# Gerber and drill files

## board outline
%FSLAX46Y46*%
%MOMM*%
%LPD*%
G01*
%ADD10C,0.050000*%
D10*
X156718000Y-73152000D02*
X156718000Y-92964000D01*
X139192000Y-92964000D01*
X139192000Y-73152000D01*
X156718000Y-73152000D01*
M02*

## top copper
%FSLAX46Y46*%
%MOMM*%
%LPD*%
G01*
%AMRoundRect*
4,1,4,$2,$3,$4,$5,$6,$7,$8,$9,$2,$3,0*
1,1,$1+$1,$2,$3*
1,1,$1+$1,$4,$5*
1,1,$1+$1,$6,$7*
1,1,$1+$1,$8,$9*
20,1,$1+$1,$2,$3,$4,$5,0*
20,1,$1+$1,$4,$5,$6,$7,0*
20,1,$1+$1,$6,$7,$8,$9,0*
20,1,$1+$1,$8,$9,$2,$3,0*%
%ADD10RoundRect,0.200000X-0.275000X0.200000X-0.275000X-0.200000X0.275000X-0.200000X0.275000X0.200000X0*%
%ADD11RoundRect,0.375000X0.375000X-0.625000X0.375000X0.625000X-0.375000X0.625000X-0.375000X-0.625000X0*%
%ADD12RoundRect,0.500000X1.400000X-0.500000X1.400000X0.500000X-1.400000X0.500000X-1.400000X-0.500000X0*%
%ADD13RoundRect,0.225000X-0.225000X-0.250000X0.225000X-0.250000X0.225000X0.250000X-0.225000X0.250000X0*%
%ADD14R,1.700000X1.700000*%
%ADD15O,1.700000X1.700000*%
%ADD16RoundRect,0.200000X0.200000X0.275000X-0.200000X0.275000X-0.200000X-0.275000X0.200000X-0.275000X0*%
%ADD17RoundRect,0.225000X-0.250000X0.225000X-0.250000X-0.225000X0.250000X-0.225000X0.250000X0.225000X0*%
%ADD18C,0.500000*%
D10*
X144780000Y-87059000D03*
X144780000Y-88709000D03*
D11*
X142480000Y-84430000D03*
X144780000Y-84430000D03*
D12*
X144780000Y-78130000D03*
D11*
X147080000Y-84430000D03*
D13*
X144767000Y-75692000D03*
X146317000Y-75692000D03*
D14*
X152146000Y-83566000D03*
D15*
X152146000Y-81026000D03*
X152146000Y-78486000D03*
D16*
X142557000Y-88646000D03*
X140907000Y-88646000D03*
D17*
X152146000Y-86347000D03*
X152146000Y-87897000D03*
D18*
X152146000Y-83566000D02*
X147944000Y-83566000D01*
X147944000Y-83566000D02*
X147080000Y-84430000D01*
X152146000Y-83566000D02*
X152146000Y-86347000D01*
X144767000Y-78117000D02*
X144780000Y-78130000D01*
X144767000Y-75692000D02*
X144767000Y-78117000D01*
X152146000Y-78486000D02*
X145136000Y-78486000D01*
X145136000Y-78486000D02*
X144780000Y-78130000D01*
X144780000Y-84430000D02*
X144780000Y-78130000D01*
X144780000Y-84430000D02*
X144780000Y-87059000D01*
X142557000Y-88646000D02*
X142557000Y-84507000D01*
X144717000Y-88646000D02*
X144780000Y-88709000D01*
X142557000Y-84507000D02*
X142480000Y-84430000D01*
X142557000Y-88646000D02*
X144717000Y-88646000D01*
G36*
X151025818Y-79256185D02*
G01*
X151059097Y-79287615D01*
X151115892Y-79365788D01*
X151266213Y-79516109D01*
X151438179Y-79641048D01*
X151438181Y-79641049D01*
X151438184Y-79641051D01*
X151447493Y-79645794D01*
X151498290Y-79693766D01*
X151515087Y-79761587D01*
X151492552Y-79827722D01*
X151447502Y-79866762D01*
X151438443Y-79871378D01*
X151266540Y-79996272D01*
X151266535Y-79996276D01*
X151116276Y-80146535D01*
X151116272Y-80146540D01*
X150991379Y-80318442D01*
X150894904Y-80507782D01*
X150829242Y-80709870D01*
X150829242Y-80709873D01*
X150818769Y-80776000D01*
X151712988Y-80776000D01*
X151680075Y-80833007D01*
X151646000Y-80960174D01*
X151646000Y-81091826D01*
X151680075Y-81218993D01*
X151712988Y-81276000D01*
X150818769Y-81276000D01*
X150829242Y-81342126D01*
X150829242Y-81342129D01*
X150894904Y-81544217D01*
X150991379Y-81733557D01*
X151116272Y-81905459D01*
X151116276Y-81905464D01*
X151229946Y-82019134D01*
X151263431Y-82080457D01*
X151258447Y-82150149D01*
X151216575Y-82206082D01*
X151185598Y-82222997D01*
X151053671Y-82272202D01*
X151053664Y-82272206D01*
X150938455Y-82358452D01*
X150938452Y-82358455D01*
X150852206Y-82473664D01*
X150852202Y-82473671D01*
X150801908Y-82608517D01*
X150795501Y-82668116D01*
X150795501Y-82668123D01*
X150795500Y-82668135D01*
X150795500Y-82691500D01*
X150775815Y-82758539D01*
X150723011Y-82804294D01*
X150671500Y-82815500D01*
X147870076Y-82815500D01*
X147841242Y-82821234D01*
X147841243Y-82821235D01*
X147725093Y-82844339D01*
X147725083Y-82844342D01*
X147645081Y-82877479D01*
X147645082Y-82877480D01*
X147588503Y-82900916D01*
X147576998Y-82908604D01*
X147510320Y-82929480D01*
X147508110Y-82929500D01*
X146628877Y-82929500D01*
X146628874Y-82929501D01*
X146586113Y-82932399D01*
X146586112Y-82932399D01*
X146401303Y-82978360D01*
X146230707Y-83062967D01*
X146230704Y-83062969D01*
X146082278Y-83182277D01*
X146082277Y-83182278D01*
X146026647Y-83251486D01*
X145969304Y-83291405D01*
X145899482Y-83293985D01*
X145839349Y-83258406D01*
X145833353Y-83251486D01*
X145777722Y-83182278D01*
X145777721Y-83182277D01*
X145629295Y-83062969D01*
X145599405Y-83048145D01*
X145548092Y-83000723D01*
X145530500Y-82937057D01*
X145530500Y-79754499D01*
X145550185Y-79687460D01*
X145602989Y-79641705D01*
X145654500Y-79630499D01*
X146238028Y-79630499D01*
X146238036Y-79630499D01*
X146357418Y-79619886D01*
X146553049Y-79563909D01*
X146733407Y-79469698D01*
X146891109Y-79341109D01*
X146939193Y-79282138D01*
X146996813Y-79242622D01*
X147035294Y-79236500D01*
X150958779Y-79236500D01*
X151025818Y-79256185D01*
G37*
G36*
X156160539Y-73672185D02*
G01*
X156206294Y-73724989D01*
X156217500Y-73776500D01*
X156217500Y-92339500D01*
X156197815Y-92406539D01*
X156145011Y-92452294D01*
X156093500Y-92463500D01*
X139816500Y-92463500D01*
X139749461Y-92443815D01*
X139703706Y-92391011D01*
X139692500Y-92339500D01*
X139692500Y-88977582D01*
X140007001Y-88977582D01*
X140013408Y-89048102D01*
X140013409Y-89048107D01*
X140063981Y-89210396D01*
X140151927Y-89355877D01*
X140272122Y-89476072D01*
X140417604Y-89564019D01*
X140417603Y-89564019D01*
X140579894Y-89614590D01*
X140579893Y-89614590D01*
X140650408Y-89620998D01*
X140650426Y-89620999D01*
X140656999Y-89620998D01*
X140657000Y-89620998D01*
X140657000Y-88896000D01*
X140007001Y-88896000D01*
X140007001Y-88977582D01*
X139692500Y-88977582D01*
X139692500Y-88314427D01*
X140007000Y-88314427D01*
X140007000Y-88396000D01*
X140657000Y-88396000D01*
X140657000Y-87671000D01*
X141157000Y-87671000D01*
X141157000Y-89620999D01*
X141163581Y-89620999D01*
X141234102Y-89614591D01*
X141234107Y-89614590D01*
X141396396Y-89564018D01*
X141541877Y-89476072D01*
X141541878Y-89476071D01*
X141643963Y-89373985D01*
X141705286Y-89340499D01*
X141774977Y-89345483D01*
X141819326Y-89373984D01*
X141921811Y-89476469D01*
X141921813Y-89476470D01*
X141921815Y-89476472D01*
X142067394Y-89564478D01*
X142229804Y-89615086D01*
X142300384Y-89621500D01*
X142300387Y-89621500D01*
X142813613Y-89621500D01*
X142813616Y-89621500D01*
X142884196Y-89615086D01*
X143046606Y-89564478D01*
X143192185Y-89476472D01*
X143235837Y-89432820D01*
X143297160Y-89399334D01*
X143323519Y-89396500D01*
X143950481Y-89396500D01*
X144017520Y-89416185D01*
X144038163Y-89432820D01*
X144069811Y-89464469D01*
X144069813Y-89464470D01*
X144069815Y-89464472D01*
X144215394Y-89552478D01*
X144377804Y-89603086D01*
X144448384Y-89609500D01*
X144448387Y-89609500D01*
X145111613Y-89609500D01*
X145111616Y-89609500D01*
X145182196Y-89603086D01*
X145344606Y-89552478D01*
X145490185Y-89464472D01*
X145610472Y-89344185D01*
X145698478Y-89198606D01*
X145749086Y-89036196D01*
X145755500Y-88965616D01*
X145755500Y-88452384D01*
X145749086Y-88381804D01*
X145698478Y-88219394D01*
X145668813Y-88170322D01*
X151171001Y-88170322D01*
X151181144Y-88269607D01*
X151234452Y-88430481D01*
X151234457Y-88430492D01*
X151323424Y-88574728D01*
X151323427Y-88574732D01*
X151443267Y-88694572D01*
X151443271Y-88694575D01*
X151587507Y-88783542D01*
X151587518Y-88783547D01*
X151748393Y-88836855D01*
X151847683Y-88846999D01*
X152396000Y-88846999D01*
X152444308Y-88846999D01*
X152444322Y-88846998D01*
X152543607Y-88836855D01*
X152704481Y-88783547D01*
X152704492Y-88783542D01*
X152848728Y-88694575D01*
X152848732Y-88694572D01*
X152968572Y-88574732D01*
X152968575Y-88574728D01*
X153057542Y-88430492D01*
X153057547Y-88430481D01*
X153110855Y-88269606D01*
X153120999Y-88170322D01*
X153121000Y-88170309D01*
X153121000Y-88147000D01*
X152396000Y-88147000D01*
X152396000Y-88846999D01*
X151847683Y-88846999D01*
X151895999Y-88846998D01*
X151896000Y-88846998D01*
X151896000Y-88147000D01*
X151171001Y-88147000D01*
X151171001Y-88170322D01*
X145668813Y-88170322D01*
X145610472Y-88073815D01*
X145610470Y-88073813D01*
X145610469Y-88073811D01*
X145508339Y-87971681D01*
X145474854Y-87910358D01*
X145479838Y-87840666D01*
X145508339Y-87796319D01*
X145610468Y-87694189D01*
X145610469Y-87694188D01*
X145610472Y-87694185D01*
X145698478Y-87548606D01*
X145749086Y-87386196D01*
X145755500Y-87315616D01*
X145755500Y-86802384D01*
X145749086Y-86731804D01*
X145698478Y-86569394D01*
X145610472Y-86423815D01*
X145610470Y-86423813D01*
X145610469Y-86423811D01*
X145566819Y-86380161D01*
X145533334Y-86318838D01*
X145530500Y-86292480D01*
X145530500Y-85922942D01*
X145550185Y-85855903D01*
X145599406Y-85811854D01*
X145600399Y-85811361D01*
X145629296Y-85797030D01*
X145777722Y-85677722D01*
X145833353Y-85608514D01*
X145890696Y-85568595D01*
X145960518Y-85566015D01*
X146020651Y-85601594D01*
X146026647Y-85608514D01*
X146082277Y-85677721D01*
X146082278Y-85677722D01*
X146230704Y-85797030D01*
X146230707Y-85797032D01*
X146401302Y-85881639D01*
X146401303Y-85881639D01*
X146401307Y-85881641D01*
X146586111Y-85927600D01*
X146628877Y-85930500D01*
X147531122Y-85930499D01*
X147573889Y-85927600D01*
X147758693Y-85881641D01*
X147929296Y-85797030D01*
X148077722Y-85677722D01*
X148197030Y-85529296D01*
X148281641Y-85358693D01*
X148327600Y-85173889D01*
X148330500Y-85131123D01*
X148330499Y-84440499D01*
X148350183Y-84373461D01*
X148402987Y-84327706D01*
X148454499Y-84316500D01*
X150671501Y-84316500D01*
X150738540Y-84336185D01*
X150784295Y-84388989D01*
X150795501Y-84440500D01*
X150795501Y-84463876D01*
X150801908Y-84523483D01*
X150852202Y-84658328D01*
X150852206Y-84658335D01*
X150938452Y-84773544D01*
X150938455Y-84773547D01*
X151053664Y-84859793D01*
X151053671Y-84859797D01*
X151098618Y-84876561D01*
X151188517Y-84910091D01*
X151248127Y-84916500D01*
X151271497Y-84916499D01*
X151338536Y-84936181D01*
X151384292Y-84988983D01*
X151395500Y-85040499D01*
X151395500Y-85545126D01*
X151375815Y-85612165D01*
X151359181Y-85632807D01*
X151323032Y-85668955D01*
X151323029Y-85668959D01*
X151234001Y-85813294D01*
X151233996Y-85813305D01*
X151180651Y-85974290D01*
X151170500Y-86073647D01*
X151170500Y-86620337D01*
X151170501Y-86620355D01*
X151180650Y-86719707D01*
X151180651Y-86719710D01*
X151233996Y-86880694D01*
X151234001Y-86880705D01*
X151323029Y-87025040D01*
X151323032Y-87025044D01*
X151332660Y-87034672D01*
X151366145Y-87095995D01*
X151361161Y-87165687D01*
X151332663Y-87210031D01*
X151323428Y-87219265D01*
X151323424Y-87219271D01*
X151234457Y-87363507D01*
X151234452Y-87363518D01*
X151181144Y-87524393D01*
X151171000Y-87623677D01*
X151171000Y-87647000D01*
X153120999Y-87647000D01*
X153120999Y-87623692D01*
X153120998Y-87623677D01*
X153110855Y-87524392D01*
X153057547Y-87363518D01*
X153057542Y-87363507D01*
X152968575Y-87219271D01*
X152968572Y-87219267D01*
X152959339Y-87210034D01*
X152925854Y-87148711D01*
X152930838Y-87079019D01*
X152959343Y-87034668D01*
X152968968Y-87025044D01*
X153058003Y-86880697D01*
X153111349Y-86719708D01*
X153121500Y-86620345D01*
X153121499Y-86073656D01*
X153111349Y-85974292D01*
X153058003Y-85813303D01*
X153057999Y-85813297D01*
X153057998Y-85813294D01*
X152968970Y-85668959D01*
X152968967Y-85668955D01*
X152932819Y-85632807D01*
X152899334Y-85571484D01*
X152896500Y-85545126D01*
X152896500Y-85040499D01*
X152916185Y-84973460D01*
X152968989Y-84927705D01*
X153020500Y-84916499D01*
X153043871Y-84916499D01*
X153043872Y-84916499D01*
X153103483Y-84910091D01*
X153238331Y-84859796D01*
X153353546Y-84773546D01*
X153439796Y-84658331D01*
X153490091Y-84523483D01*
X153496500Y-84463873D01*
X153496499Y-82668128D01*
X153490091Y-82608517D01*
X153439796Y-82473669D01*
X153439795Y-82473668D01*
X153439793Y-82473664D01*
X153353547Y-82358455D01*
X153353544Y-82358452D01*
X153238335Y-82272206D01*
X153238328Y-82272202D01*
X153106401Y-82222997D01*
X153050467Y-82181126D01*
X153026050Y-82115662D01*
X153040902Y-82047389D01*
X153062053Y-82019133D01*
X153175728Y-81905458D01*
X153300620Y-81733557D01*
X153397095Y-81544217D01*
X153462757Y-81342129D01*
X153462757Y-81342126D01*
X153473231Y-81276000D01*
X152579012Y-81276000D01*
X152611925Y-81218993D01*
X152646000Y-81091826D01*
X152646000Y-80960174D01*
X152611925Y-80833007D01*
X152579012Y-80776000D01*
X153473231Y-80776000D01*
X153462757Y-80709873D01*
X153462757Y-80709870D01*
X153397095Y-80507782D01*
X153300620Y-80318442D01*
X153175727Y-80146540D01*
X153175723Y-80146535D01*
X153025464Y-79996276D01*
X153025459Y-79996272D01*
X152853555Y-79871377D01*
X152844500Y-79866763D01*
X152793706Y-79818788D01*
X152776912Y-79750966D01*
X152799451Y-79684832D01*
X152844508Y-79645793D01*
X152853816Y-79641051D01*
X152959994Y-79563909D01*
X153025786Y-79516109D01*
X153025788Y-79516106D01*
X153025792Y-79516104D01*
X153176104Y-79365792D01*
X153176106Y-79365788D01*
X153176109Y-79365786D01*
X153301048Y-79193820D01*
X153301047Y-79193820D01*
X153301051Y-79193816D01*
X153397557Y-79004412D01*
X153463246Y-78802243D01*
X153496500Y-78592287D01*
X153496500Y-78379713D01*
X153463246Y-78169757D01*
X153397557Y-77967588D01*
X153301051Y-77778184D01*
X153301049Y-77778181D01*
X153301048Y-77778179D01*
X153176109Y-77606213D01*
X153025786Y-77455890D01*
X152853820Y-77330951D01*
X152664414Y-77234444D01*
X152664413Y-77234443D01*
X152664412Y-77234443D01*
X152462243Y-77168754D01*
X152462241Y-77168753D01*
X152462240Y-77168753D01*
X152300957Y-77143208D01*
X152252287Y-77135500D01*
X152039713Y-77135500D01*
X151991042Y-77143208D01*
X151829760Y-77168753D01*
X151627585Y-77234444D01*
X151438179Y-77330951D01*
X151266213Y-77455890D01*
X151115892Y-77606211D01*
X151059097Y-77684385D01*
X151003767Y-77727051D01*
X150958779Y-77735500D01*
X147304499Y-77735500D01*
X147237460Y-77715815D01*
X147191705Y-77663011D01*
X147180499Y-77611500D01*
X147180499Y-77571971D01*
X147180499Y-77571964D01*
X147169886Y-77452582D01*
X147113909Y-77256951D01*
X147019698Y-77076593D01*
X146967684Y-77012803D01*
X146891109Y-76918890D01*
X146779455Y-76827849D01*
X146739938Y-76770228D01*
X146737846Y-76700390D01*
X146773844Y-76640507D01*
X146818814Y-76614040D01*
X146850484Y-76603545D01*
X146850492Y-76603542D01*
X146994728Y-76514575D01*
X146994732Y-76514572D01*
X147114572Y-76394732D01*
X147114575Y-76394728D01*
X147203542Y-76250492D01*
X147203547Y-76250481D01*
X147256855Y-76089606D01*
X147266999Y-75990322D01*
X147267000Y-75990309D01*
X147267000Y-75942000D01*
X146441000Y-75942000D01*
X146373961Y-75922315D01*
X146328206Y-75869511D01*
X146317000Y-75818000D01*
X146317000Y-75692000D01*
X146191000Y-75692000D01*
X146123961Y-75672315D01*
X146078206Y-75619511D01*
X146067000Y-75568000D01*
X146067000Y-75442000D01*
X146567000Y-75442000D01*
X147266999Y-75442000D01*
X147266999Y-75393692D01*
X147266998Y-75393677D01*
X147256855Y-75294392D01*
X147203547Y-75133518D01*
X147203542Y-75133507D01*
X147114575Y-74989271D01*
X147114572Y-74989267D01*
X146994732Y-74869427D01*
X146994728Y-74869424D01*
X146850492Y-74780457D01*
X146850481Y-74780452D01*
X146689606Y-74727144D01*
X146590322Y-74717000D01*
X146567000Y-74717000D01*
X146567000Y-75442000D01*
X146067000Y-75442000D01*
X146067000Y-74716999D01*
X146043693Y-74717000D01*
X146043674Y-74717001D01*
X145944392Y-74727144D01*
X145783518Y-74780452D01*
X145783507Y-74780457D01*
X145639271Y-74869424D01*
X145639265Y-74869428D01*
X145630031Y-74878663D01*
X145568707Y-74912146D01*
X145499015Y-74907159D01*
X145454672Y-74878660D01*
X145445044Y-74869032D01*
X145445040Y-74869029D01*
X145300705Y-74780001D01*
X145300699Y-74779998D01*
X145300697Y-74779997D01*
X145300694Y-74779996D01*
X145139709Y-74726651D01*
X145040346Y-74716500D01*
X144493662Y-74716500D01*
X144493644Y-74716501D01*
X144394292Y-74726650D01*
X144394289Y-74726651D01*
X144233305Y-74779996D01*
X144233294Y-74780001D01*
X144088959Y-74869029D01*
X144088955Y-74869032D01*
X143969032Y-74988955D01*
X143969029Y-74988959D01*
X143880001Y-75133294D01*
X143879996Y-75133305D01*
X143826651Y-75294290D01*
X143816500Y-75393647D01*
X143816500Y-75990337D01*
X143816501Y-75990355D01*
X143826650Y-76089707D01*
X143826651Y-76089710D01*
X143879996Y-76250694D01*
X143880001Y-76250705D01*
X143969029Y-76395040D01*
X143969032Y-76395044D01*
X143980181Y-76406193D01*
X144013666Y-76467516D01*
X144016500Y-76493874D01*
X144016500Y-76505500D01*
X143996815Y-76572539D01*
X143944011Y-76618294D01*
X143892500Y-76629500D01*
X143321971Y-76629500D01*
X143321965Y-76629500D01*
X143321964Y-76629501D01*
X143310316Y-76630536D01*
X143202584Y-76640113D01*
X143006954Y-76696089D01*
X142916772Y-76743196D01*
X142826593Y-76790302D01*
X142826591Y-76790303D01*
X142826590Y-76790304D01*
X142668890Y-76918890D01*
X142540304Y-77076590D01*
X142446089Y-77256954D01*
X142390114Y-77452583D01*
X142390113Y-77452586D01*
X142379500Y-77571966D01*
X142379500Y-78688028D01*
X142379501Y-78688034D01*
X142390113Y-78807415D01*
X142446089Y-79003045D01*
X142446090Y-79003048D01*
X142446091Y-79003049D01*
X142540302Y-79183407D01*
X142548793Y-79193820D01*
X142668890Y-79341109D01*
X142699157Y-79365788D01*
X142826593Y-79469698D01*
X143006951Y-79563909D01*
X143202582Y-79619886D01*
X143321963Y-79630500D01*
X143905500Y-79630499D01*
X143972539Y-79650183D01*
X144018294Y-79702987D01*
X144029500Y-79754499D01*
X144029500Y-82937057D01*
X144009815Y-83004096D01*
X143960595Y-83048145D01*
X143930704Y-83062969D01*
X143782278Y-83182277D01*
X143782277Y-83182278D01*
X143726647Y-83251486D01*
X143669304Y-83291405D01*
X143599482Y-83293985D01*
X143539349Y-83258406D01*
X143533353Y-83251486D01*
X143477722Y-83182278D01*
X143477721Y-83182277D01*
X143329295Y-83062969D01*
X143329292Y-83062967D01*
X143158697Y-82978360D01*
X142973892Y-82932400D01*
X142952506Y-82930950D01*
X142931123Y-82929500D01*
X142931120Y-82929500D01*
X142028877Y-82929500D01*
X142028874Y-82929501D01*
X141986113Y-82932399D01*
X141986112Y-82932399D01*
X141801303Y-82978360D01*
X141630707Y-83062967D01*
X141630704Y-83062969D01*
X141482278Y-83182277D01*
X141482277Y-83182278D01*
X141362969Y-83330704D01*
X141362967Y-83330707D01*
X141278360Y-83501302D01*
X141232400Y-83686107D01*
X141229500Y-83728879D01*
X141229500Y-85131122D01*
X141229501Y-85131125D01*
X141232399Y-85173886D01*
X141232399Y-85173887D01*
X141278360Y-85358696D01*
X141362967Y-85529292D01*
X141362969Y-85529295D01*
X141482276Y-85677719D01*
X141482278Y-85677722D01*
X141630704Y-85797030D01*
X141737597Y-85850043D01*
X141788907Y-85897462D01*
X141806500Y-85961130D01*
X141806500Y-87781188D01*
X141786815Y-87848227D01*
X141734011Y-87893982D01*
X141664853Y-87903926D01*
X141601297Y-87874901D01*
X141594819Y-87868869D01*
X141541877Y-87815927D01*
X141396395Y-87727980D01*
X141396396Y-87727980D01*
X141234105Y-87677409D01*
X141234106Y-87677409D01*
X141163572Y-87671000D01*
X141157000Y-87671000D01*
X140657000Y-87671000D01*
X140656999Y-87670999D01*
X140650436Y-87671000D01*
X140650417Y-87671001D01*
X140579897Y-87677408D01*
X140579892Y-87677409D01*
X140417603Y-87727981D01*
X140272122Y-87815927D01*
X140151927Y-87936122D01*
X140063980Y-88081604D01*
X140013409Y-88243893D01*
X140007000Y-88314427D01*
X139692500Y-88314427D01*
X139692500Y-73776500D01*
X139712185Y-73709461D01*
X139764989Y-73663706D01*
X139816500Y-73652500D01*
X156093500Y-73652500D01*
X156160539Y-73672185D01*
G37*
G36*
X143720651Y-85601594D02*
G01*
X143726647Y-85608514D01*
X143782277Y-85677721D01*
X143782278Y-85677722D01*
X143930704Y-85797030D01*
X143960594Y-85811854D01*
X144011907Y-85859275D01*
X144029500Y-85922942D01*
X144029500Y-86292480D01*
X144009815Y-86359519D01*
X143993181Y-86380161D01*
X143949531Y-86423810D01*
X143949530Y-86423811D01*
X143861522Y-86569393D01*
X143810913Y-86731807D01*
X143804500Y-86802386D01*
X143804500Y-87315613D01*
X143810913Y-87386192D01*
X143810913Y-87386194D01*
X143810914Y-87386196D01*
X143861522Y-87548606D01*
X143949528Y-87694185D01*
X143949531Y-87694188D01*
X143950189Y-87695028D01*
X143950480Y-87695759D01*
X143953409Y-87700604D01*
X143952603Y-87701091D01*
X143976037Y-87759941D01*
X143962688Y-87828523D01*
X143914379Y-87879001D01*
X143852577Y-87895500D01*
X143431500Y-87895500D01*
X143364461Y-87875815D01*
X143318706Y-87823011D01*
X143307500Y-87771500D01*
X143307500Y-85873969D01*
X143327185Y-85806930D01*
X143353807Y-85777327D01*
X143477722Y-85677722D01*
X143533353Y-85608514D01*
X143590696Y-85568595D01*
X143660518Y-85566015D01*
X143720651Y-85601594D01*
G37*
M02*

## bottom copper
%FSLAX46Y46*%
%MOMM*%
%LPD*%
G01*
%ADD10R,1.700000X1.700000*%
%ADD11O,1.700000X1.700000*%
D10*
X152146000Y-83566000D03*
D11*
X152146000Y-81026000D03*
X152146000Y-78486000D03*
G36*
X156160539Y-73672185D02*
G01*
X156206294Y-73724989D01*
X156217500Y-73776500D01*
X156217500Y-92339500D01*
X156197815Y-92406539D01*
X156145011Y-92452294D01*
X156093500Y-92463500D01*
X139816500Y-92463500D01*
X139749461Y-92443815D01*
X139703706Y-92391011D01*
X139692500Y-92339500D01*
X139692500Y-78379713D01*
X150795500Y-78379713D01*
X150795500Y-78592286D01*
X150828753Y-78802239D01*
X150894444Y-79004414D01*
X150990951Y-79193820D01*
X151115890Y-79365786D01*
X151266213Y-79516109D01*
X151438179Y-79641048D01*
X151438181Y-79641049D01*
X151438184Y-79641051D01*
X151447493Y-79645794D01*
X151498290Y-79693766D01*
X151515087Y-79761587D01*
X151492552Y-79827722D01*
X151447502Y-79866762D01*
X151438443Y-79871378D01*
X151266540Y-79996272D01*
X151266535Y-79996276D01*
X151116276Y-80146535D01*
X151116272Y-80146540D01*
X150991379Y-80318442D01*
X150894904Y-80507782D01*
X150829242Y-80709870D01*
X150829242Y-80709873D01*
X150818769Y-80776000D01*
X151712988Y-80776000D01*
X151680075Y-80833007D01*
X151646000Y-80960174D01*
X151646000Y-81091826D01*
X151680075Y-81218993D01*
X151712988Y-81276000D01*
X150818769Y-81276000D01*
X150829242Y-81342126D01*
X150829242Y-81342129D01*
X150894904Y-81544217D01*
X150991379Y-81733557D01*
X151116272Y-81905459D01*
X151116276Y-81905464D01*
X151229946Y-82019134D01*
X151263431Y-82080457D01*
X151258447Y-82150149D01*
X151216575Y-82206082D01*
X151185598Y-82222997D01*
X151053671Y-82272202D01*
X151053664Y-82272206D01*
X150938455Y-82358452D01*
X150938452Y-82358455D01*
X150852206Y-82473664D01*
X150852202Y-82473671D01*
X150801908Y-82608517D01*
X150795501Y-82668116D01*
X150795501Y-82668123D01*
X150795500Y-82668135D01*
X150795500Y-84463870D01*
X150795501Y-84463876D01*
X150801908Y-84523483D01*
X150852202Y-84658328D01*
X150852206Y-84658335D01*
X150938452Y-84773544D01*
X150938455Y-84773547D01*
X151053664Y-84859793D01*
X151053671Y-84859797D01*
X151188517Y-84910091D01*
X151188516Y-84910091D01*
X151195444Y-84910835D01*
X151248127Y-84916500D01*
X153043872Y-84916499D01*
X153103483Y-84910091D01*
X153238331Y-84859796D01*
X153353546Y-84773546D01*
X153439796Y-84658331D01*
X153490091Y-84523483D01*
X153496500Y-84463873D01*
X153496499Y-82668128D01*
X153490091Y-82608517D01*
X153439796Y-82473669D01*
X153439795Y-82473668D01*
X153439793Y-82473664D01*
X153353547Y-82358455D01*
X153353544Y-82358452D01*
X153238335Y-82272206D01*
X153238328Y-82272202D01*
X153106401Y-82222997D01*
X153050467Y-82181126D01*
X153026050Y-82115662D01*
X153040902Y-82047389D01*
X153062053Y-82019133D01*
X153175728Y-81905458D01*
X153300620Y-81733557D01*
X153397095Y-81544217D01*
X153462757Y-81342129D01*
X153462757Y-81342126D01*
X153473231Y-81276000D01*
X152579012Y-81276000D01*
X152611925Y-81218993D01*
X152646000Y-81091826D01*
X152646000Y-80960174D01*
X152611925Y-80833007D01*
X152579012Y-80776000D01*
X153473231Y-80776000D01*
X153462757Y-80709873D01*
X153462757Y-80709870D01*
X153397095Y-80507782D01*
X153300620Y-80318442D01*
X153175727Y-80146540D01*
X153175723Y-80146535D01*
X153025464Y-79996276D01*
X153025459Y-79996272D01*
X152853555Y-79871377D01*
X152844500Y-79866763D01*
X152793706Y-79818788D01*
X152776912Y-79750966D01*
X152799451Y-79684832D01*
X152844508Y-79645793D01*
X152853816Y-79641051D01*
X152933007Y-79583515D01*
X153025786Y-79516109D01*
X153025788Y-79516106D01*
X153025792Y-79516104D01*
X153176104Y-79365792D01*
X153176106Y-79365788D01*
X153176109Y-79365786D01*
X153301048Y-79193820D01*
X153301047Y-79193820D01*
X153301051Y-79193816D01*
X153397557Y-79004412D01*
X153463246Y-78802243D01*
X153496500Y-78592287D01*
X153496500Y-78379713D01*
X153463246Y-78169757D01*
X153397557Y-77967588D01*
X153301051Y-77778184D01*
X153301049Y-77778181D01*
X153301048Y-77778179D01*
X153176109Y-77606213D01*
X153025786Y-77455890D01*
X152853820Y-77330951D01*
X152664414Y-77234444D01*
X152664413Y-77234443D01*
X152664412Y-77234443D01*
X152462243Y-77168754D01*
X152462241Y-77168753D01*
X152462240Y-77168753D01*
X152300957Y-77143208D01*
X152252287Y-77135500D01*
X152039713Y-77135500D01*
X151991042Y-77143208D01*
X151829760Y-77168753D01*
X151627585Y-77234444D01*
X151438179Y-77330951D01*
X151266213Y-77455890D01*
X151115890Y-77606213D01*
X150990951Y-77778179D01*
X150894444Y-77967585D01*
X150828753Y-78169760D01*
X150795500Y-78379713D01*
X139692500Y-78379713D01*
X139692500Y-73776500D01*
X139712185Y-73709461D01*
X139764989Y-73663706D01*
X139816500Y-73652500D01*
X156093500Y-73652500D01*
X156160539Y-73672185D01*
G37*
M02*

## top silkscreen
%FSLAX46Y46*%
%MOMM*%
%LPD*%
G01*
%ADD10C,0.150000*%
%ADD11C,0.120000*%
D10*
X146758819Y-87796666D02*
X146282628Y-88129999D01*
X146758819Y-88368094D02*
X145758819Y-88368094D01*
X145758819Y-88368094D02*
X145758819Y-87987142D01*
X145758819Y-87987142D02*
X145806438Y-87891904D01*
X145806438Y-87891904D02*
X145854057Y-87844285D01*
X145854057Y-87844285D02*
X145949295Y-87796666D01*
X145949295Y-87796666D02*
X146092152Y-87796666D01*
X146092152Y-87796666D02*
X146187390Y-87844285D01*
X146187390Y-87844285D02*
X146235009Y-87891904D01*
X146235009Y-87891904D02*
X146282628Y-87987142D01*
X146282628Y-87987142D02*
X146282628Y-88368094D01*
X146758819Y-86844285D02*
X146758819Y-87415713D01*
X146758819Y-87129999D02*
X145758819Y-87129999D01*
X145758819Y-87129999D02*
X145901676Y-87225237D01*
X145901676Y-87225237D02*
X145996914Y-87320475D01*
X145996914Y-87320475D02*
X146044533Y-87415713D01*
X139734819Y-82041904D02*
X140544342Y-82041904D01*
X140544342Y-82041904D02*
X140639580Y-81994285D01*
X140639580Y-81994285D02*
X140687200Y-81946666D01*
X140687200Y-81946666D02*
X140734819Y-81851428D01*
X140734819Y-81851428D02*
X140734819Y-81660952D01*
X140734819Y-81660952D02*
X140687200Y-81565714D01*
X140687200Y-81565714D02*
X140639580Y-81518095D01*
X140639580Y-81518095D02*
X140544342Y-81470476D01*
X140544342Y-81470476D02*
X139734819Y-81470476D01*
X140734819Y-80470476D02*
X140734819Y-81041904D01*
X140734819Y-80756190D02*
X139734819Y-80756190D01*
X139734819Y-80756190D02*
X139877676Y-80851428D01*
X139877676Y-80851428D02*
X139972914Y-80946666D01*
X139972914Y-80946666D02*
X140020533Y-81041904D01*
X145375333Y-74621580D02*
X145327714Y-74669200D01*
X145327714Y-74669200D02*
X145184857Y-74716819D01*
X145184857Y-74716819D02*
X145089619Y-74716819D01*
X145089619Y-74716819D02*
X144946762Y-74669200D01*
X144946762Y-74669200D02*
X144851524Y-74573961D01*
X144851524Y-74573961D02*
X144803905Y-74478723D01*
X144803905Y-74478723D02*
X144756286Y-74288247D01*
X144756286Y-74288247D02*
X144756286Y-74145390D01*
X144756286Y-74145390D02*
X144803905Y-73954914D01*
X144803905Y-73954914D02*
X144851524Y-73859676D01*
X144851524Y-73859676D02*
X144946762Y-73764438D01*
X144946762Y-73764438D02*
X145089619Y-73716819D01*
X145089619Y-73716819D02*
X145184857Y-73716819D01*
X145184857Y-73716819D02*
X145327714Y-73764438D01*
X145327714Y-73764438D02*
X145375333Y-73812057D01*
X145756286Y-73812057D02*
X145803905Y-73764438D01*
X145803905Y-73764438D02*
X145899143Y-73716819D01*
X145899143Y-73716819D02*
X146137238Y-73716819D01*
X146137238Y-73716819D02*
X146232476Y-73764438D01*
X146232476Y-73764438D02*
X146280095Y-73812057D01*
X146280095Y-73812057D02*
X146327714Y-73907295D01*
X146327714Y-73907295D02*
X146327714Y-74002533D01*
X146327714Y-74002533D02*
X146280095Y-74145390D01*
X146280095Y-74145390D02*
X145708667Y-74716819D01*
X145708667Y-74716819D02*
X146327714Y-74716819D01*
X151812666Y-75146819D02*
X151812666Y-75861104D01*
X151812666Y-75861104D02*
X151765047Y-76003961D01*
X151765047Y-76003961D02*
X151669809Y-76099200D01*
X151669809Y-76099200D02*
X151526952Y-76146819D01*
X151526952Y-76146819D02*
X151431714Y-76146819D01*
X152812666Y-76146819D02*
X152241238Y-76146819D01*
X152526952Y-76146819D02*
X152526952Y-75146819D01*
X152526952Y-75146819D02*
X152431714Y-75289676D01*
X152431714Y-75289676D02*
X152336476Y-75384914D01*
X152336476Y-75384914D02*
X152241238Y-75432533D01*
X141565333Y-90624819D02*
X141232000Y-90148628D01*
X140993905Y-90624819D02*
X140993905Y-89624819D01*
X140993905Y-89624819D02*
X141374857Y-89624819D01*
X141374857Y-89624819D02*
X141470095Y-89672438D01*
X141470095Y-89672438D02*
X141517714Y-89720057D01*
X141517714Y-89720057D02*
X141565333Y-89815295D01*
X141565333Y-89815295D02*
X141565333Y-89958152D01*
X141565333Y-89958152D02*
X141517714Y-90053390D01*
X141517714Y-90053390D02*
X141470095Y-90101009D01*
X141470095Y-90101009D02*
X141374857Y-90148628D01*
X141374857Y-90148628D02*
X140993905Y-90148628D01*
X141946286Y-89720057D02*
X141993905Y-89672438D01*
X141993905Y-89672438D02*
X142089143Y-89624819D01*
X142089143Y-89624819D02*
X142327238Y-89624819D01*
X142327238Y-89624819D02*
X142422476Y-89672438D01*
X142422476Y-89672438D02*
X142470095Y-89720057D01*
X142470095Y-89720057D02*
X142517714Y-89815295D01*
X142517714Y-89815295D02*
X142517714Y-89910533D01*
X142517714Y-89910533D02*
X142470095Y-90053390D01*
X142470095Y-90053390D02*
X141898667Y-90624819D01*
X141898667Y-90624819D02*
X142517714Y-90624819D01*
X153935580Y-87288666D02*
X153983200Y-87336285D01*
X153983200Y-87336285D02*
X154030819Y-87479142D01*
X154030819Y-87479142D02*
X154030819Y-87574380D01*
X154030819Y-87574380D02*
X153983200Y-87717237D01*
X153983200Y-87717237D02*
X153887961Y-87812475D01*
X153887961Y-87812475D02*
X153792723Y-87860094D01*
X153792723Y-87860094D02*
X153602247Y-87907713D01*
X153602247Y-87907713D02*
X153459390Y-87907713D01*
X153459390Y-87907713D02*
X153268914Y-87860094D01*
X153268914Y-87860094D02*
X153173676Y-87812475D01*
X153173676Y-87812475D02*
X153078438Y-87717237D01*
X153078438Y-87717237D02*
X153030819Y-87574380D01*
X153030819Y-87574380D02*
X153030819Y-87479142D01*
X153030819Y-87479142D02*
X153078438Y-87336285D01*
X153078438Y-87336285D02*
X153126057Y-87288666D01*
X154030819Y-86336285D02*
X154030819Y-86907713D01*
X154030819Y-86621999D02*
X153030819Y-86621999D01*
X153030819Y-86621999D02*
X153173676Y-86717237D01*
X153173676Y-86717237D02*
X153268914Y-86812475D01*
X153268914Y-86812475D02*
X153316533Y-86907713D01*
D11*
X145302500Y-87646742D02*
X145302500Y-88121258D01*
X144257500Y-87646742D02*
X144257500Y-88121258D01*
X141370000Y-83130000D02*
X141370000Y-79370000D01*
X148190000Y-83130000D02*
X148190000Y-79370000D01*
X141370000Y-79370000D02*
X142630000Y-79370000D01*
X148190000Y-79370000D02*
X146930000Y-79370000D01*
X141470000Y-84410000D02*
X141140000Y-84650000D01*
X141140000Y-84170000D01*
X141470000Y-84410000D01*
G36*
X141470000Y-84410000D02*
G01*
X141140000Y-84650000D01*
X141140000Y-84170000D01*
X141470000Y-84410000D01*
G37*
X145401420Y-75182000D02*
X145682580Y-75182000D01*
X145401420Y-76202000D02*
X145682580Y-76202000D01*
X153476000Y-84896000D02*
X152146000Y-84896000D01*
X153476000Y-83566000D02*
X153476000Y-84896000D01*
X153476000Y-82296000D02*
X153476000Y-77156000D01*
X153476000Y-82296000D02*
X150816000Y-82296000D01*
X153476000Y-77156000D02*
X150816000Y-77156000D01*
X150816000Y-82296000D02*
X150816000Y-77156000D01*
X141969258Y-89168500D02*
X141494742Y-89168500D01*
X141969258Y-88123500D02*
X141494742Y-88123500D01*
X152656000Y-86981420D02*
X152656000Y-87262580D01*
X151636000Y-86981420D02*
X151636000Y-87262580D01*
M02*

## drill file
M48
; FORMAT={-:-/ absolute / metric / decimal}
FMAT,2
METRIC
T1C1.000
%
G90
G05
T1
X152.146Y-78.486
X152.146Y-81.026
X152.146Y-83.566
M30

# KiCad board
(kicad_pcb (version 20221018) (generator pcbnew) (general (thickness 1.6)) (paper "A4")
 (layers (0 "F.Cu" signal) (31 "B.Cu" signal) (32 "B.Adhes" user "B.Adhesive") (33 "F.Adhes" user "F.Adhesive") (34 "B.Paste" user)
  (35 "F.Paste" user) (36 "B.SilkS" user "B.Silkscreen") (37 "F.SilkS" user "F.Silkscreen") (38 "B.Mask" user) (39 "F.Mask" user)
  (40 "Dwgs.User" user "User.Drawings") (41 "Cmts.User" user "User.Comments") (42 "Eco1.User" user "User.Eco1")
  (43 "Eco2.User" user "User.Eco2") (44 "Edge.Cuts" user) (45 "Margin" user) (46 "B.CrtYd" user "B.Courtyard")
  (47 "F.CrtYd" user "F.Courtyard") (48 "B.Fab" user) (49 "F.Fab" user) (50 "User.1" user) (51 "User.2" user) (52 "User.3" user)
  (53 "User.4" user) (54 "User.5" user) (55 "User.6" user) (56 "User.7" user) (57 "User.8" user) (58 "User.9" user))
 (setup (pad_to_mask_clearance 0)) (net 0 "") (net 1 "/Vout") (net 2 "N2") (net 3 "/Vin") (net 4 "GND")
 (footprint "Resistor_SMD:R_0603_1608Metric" (layer "F.Cu") (at 144.78 87.884 -90)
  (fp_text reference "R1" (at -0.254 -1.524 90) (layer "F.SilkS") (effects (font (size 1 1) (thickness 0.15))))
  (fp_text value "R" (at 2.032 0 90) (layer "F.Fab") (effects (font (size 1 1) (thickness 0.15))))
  (fp_line (start -0.237258 -0.5225) (end 0.237258 -0.5225) (stroke (width 0.12) (type solid)) (layer "F.SilkS"))
  (fp_line (start -0.237258 0.5225) (end 0.237258 0.5225) (stroke (width 0.12) (type solid)) (layer "F.SilkS"))
  (pad "1" smd roundrect (at -0.825 0 270) (size 0.8 0.95) (layers "F.Cu" "F.Paste" "F.Mask") (roundrect_rratio 0.25) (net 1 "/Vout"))
  (pad "2" smd roundrect (at 0.825 0 270) (size 0.8 0.95) (layers "F.Cu" "F.Paste" "F.Mask") (roundrect_rratio 0.25) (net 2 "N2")))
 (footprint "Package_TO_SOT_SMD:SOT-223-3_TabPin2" (layer "F.Cu") (at 144.78 81.28 90)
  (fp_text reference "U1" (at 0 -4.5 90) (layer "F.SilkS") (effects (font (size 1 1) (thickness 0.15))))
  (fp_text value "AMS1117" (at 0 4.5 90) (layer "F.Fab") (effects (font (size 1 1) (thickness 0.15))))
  (fp_line (start -1.85 -3.41) (end 1.91 -3.41) (stroke (width 0.12) (type solid)) (layer "F.SilkS"))
  (fp_line (start -1.85 3.41) (end 1.91 3.41) (stroke (width 0.12) (type solid)) (layer "F.SilkS"))
  (fp_line (start 1.91 -3.41) (end 1.91 -2.15) (stroke (width 0.12) (type solid)) (layer "F.SilkS"))
  (fp_line (start 1.91 3.41) (end 1.91 2.15) (stroke (width 0.12) (type solid)) (layer "F.SilkS"))
  (fp_poly
   (pts (xy -3.13 -3.31) (xy -3.37 -3.64) (xy -2.89 -3.64) (xy -3.13 -3.31)) (stroke (width 0.12) (type solid)) (fill solid)
   (layer "F.SilkS"))
  (pad "1" smd roundrect (at -3.15 -2.3 90) (size 2 1.5) (layers "F.Cu" "F.Paste" "F.Mask") (roundrect_rratio 0.25) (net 2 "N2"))
  (pad "2" smd roundrect (at -3.15 0 90) (size 2 1.5) (layers "F.Cu" "F.Paste" "F.Mask") (roundrect_rratio 0.25) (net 1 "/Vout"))
  (pad "2" smd roundrect (at 3.15 0 90) (size 2 3.8) (layers "F.Cu" "F.Paste" "F.Mask") (roundrect_rratio 0.25) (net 1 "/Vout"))
  (pad "3" smd roundrect (at -3.15 2.3 90) (size 2 1.5) (layers "F.Cu" "F.Paste" "F.Mask") (roundrect_rratio 0.25) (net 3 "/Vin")))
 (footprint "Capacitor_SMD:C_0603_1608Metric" (layer "F.Cu") (at 145.542 75.692)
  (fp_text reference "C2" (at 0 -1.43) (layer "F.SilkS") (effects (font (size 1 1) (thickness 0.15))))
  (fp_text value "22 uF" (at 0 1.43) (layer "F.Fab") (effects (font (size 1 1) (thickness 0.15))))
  (fp_line (start -0.14058 -0.51) (end 0.14058 -0.51) (stroke (width 0.12) (type solid)) (layer "F.SilkS"))
  (fp_line (start -0.14058 0.51) (end 0.14058 0.51) (stroke (width 0.12) (type solid)) (layer "F.SilkS"))
  (pad "1" smd roundrect (at -0.775 0) (size 0.9 0.95) (layers "F.Cu" "F.Paste" "F.Mask") (roundrect_rratio 0.25) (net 1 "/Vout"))
  (pad "2" smd roundrect (at 0.775 0) (size 0.9 0.95) (layers "F.Cu" "F.Paste" "F.Mask") (roundrect_rratio 0.25) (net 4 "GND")))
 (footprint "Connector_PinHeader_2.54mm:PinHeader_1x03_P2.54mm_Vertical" (layer "F.Cu") (at 152.146 83.566 180)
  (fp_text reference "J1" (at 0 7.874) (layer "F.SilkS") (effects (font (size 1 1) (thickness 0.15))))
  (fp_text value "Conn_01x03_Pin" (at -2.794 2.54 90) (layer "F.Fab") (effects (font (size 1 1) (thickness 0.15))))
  (fp_line (start -1.33 -1.33) (end 0 -1.33) (stroke (width 0.12) (type solid)) (layer "F.SilkS"))
  (fp_line (start -1.33 0) (end -1.33 -1.33) (stroke (width 0.12) (type solid)) (layer "F.SilkS"))
  (fp_line (start -1.33 1.27) (end -1.33 6.41) (stroke (width 0.12) (type solid)) (layer "F.SilkS"))
  (fp_line (start -1.33 1.27) (end 1.33 1.27) (stroke (width 0.12) (type solid)) (layer "F.SilkS"))
  (fp_line (start -1.33 6.41) (end 1.33 6.41) (stroke (width 0.12) (type solid)) (layer "F.SilkS"))
  (fp_line (start 1.33 1.27) (end 1.33 6.41) (stroke (width 0.12) (type solid)) (layer "F.SilkS"))
  (pad "1" thru_hole rect (at 0 0 180) (size 1.7 1.7) (drill 1) (layers "*.Cu" "*.Mask") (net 3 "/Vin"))
  (pad "2" thru_hole oval (at 0 2.54 180) (size 1.7 1.7) (drill 1) (layers "*.Cu" "*.Mask") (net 4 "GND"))
  (pad "3" thru_hole oval (at 0 5.08 180) (size 1.7 1.7) (drill 1) (layers "*.Cu" "*.Mask") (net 1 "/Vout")))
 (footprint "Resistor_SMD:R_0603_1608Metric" (layer "F.Cu") (at 141.732 88.646 180)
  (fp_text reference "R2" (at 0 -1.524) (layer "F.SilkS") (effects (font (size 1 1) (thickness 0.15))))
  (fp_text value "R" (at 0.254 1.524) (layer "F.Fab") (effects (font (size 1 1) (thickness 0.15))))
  (fp_line (start -0.237258 -0.5225) (end 0.237258 -0.5225) (stroke (width 0.12) (type solid)) (layer "F.SilkS"))
  (fp_line (start -0.237258 0.5225) (end 0.237258 0.5225) (stroke (width 0.12) (type solid)) (layer "F.SilkS"))
  (pad "1" smd roundrect (at -0.825 0 180) (size 0.8 0.95) (layers "F.Cu" "F.Paste" "F.Mask") (roundrect_rratio 0.25) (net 2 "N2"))
  (pad "2" smd roundrect (at 0.825 0 180) (size 0.8 0.95) (layers "F.Cu" "F.Paste" "F.Mask") (roundrect_rratio 0.25) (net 4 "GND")))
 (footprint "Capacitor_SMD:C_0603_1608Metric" (layer "F.Cu") (at 152.146 87.122 -90)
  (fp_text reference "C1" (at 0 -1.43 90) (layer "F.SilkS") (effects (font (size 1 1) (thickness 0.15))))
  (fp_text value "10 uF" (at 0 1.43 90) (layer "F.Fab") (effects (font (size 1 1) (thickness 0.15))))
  (fp_line (start -0.14058 -0.51) (end 0.14058 -0.51) (stroke (width 0.12) (type solid)) (layer "F.SilkS"))
  (fp_line (start -0.14058 0.51) (end 0.14058 0.51) (stroke (width 0.12) (type solid)) (layer "F.SilkS"))
  (pad "1" smd roundrect (at -0.775 0 270) (size 0.9 0.95) (layers "F.Cu" "F.Paste" "F.Mask") (roundrect_rratio 0.25) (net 3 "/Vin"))
  (pad "2" smd roundrect (at 0.775 0 270) (size 0.9 0.95) (layers "F.Cu" "F.Paste" "F.Mask") (roundrect_rratio 0.25) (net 4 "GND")))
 (gr_poly
  (pts (xy 156.718 73.152) (xy 156.718 92.964) (xy 139.192 92.964) (xy 139.192 73.152)) (stroke (width 0.05) (type solid)) (fill none)
  (layer "Edge.Cuts"))
 (segment (start 152.146 83.566) (end 147.944 83.566) (width 0.5) (layer "F.Cu") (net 3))
 (segment (start 147.944 83.566) (end 147.08 84.43) (width 0.5) (layer "F.Cu") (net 3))
 (segment (start 152.146 83.566) (end 152.146 86.347) (width 0.5) (layer "F.Cu") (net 3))
 (segment (start 144.767 78.117) (end 144.78 78.13) (width 0.5) (layer "F.Cu") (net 1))
 (segment (start 144.767 75.692) (end 144.767 78.117) (width 0.5) (layer "F.Cu") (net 1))
 (segment (start 152.146 78.486) (end 145.136 78.486) (width 0.5) (layer "F.Cu") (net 1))
 (segment (start 145.136 78.486) (end 144.78 78.13) (width 0.5) (layer "F.Cu") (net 1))
 (segment (start 144.78 84.43) (end 144.78 78.13) (width 0.5) (layer "F.Cu") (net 1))
 (segment (start 144.78 84.43) (end 144.78 87.059) (width 0.5) (layer "F.Cu") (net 1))
 (segment (start 142.557 88.646) (end 142.557 84.507) (width 0.5) (layer "F.Cu") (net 2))
 (segment (start 144.717 88.646) (end 144.78 88.709) (width 0.5) (layer "F.Cu") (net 2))
 (segment (start 142.557 84.507) (end 142.48 84.43) (width 0.5) (layer "F.Cu") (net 2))
 (segment (start 142.557 88.646) (end 144.717 88.646) (width 0.5) (layer "F.Cu") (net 2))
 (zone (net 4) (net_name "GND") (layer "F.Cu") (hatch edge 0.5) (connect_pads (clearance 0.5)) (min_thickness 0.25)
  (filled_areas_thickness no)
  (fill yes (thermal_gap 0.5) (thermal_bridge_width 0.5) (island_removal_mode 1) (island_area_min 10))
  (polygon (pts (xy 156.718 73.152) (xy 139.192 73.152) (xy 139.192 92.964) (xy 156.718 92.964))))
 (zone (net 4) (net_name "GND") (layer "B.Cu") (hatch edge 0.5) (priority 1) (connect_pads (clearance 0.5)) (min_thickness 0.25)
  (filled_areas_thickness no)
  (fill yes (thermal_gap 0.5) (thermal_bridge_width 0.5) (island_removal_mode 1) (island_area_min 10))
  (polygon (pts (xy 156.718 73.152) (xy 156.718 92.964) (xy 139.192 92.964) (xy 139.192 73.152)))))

